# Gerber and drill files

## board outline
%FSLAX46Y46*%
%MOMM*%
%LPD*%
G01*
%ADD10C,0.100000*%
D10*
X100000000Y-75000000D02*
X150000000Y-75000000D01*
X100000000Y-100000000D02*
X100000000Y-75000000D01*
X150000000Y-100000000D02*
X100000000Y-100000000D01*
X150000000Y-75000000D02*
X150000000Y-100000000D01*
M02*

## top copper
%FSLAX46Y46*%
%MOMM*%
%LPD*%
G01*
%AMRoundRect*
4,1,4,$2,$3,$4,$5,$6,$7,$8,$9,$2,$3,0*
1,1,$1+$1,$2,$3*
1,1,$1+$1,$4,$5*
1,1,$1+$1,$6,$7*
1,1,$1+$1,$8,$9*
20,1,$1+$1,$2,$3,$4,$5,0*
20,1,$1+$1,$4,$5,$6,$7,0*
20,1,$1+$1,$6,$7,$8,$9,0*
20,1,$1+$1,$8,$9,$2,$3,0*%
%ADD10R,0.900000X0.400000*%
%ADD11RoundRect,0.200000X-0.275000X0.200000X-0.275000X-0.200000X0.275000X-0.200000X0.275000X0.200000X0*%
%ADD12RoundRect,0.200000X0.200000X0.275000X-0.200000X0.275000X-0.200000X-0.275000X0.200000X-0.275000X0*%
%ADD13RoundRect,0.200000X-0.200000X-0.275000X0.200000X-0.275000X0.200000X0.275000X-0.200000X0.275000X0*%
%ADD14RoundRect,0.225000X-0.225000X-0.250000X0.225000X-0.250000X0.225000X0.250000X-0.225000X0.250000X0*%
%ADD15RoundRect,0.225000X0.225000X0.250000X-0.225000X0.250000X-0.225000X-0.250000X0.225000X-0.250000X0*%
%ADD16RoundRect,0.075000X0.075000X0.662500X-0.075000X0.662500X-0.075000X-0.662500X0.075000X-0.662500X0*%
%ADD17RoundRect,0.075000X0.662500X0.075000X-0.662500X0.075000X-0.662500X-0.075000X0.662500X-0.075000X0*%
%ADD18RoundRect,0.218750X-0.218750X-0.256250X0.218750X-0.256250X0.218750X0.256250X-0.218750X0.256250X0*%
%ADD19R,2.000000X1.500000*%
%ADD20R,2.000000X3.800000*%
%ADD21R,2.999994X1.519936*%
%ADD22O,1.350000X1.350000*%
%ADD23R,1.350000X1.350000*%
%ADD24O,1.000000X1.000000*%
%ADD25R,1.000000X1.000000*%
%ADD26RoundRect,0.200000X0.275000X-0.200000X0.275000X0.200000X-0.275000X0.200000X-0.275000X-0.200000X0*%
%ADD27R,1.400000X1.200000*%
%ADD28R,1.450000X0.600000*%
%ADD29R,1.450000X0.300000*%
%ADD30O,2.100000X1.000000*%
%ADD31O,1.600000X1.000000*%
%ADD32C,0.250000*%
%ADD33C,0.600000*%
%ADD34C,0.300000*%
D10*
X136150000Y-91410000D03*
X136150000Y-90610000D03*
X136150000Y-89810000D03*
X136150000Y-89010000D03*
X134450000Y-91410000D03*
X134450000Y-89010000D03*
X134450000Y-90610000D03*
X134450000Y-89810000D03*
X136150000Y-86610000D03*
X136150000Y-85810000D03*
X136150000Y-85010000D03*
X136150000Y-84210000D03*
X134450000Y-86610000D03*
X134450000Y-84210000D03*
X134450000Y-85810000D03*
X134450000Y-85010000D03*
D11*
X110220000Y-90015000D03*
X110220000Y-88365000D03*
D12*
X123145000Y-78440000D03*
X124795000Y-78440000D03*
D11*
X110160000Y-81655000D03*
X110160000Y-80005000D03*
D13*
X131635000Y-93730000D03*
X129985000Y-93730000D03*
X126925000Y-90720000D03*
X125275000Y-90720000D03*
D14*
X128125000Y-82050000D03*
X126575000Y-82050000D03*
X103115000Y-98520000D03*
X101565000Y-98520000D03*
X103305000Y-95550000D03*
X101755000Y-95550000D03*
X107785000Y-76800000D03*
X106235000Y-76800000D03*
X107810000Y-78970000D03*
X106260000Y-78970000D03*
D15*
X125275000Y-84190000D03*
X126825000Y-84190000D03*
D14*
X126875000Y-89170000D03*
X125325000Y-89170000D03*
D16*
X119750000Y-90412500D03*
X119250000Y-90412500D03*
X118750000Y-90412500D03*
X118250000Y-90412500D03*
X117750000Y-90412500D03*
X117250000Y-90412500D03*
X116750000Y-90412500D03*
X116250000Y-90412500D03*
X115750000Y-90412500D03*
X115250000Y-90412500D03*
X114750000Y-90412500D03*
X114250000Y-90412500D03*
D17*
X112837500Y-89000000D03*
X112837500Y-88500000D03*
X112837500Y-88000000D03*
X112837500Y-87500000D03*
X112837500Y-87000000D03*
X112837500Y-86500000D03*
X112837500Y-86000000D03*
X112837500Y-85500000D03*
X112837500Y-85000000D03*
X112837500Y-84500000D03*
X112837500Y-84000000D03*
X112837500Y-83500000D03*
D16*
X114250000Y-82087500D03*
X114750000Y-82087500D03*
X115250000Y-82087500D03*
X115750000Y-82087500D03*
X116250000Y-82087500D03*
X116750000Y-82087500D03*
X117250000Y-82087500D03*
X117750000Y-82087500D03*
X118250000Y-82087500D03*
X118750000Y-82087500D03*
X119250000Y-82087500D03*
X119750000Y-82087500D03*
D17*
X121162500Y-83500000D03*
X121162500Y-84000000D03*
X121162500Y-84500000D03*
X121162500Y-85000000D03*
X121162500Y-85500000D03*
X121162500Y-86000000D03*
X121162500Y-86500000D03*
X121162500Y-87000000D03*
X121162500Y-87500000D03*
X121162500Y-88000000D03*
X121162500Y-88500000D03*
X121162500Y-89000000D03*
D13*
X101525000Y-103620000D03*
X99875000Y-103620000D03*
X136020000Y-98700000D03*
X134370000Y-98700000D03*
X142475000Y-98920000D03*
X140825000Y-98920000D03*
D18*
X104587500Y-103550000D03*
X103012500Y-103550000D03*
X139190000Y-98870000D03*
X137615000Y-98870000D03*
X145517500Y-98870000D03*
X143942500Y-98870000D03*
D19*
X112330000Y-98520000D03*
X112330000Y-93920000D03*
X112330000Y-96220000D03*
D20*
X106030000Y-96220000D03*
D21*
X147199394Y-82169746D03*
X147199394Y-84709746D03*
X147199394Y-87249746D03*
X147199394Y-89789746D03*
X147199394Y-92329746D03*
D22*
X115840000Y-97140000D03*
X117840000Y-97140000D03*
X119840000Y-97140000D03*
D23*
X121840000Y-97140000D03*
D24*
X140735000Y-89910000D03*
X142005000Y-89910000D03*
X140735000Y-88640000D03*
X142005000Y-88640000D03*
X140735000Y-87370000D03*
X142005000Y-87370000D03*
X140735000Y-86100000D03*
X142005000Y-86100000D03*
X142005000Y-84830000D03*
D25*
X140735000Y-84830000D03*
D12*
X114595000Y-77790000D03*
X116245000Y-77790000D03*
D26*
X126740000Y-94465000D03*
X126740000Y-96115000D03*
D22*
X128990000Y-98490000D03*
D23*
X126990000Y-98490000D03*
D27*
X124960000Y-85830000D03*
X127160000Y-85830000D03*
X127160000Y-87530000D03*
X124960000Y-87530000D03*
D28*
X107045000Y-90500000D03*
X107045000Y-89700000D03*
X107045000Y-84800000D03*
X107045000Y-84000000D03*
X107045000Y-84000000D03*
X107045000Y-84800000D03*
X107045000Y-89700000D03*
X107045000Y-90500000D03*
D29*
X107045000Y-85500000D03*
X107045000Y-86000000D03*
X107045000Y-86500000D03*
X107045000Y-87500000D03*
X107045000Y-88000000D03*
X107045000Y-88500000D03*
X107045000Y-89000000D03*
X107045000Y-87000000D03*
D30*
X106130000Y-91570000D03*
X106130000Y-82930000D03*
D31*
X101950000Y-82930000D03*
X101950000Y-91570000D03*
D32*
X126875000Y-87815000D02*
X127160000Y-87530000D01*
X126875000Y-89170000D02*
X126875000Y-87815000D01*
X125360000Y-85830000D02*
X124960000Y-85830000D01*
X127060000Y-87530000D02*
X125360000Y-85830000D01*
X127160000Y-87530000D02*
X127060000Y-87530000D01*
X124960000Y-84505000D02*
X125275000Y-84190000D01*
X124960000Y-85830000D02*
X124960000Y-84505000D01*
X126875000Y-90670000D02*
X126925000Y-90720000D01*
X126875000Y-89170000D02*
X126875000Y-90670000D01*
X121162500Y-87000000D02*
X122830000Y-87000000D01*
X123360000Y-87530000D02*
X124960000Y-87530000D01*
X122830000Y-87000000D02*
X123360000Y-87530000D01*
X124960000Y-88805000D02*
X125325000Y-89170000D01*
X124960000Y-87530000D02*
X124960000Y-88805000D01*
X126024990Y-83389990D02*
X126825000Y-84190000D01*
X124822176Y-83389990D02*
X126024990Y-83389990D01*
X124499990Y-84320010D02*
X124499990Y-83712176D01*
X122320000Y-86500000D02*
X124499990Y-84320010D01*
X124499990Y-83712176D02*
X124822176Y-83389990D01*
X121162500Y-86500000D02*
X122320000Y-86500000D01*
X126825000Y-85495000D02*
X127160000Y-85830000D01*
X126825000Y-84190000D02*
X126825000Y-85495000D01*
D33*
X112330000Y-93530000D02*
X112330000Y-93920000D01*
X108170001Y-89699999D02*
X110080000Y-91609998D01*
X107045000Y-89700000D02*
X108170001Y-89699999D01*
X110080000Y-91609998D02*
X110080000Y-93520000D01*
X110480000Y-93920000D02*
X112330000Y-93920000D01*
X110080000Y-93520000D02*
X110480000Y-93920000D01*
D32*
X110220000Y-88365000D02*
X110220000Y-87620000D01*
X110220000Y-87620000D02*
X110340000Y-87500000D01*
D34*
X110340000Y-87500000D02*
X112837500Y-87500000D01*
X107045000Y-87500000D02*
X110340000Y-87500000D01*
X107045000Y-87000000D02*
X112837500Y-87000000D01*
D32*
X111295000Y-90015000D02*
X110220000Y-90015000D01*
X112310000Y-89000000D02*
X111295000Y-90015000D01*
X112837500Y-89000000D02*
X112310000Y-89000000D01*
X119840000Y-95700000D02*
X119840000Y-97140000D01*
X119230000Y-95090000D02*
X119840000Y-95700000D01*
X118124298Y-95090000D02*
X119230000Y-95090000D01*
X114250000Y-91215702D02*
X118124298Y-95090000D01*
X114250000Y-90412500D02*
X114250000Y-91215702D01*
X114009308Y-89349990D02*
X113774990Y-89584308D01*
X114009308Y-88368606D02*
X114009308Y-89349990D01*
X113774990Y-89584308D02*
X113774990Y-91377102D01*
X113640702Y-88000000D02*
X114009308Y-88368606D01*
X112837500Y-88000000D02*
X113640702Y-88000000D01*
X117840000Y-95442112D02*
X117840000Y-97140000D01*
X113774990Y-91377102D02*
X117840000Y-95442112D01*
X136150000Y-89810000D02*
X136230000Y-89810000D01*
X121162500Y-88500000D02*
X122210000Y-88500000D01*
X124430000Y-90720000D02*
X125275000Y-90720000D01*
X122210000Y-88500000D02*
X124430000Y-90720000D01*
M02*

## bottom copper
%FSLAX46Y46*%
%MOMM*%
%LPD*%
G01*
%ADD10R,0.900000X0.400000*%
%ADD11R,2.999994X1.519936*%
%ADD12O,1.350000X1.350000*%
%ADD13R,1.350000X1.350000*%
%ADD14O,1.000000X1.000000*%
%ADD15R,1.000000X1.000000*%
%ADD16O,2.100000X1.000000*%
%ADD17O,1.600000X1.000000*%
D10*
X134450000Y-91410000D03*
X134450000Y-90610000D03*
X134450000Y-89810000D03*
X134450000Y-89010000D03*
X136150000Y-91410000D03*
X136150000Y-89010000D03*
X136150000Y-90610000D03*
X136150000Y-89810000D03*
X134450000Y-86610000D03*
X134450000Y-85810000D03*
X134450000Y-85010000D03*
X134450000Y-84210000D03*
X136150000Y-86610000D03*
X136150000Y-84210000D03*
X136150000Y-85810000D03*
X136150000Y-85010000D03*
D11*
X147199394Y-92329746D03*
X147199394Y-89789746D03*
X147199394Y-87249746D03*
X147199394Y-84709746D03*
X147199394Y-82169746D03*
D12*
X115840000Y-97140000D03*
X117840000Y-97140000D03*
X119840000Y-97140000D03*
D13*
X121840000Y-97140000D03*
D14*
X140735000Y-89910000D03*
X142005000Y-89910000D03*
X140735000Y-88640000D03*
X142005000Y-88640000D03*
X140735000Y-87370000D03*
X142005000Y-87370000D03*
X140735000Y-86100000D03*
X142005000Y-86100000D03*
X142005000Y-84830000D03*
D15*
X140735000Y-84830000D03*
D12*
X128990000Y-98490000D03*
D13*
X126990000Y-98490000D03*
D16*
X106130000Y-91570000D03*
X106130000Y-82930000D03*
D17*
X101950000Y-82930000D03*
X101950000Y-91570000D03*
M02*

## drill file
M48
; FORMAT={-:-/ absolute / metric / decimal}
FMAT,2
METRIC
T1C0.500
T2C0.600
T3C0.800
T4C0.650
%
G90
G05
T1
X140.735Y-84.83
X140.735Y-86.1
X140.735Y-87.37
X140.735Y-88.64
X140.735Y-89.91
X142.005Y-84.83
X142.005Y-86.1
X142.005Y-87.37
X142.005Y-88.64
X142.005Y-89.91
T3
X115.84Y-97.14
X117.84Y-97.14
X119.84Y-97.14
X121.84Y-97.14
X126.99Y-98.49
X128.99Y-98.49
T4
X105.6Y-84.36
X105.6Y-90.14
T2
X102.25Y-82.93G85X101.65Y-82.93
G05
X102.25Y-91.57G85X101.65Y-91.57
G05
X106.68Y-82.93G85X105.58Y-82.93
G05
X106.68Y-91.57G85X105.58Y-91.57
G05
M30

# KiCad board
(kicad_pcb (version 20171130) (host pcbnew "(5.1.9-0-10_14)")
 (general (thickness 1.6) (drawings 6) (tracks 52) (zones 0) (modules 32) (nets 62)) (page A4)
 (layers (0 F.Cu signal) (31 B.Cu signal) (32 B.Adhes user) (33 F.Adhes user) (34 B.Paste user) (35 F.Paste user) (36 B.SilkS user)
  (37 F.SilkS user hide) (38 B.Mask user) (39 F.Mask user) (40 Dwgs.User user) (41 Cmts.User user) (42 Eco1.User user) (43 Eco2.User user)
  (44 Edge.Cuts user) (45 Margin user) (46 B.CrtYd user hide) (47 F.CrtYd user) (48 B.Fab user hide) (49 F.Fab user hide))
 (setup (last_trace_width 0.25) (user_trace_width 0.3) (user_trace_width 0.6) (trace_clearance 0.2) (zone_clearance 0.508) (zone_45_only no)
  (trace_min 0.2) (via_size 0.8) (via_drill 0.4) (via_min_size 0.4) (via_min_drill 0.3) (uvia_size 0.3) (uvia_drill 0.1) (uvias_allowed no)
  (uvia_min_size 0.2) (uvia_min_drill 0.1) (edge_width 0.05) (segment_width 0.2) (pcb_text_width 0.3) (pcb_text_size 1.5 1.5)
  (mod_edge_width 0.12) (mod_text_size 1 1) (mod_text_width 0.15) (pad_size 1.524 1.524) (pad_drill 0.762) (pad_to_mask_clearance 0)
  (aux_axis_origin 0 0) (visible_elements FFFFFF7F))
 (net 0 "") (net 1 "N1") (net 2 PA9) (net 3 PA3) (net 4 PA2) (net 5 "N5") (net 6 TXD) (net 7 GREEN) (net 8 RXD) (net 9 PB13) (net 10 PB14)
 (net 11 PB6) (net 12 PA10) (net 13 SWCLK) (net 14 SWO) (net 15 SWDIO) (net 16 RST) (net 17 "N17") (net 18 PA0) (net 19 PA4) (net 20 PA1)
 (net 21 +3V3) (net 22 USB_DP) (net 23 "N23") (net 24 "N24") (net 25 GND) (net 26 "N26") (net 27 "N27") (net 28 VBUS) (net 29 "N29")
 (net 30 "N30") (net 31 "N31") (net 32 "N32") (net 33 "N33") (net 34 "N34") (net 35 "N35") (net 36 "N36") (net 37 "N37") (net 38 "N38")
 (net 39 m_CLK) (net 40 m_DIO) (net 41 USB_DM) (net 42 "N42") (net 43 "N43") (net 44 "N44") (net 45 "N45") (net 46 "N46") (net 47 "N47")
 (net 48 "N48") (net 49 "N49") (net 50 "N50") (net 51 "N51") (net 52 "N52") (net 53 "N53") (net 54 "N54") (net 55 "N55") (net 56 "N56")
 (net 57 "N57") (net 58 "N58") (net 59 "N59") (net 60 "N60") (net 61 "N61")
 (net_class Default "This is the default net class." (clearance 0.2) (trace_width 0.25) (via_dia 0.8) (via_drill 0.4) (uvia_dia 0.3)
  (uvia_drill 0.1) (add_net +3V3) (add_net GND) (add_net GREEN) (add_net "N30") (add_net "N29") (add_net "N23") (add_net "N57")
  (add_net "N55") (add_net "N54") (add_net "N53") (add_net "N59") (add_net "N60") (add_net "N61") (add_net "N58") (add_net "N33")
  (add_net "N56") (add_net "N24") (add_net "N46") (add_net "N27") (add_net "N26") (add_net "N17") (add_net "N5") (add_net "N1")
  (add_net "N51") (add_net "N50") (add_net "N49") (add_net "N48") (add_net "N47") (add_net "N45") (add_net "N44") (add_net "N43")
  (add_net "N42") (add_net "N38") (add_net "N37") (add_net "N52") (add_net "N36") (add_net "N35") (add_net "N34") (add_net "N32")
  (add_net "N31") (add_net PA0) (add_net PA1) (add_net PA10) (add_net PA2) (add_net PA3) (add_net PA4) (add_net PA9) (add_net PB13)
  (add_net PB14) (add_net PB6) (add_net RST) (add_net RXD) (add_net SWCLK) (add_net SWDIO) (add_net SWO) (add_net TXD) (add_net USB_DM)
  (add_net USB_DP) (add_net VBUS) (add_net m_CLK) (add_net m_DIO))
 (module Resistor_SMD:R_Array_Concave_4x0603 (layer B.Cu) (at 135.3 90.21 180)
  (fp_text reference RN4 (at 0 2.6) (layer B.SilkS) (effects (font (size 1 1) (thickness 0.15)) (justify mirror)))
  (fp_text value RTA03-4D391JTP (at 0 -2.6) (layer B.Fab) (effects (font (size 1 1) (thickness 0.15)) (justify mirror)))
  (pad 5 smd rect (at 0.85 -1.2 180) (size 0.9 0.4) (layers B.Cu B.Paste B.Mask) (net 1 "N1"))
  (pad 6 smd rect (at 0.85 -0.4 180) (size 0.9 0.4) (layers B.Cu B.Paste B.Mask) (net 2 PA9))
  (pad 7 smd rect (at 0.85 0.4 180) (size 0.9 0.4) (layers B.Cu B.Paste B.Mask) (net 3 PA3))
  (pad 8 smd rect (at 0.85 1.2 180) (size 0.9 0.4) (layers B.Cu B.Paste B.Mask) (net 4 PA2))
  (pad 4 smd rect (at -0.85 -1.2 180) (size 0.9 0.4) (layers B.Cu B.Paste B.Mask) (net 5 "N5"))
  (pad 1 smd rect (at -0.85 1.2 180) (size 0.9 0.4) (layers B.Cu B.Paste B.Mask) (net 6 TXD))
  (pad 3 smd rect (at -0.85 -0.4 180) (size 0.9 0.4) (layers B.Cu B.Paste B.Mask) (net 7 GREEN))
  (pad 2 smd rect (at -0.85 0.4 180) (size 0.9 0.4) (layers B.Cu B.Paste B.Mask) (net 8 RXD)))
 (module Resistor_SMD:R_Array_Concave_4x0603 (layer B.Cu) (at 135.3 85.41 180)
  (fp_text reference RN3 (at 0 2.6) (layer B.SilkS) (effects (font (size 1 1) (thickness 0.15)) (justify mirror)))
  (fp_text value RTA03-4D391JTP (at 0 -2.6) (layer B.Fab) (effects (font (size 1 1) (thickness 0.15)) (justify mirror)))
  (pad 5 smd rect (at 0.85 -1.2 180) (size 0.9 0.4) (layers B.Cu B.Paste B.Mask) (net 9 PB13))
  (pad 6 smd rect (at 0.85 -0.4 180) (size 0.9 0.4) (layers B.Cu B.Paste B.Mask) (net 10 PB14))
  (pad 7 smd rect (at 0.85 0.4 180) (size 0.9 0.4) (layers B.Cu B.Paste B.Mask) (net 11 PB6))
  (pad 8 smd rect (at 0.85 1.2 180) (size 0.9 0.4) (layers B.Cu B.Paste B.Mask) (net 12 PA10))
  (pad 4 smd rect (at -0.85 -1.2 180) (size 0.9 0.4) (layers B.Cu B.Paste B.Mask) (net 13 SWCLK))
  (pad 1 smd rect (at -0.85 1.2 180) (size 0.9 0.4) (layers B.Cu B.Paste B.Mask) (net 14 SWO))
  (pad 3 smd rect (at -0.85 -0.4 180) (size 0.9 0.4) (layers B.Cu B.Paste B.Mask) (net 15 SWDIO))
  (pad 2 smd rect (at -0.85 0.4 180) (size 0.9 0.4) (layers B.Cu B.Paste B.Mask) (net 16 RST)))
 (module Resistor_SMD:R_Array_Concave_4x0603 (layer F.Cu) (at 135.3 90.21)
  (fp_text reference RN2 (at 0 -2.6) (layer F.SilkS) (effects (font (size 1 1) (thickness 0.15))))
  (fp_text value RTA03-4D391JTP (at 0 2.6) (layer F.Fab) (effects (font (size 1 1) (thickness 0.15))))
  (pad 5 smd rect (at 0.85 1.2) (size 0.9 0.4) (layers F.Cu F.Paste F.Mask) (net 5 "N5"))
  (pad 6 smd rect (at 0.85 0.4) (size 0.9 0.4) (layers F.Cu F.Paste F.Mask) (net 7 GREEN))
  (pad 7 smd rect (at 0.85 -0.4) (size 0.9 0.4) (layers F.Cu F.Paste F.Mask) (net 8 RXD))
  (pad 8 smd rect (at 0.85 -1.2) (size 0.9 0.4) (layers F.Cu F.Paste F.Mask) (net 6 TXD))
  (pad 4 smd rect (at -0.85 1.2) (size 0.9 0.4) (layers F.Cu F.Paste F.Mask) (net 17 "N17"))
  (pad 1 smd rect (at -0.85 -1.2) (size 0.9 0.4) (layers F.Cu F.Paste F.Mask) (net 2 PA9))
  (pad 3 smd rect (at -0.85 0.4) (size 0.9 0.4) (layers F.Cu F.Paste F.Mask) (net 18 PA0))
  (pad 2 smd rect (at -0.85 -0.4) (size 0.9 0.4) (layers F.Cu F.Paste F.Mask) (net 12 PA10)))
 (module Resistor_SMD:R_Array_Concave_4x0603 (layer F.Cu) (at 135.3 85.41)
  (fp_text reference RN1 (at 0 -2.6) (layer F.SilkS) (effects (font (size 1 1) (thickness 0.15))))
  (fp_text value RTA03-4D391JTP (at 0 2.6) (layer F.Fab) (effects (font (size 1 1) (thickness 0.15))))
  (pad 5 smd rect (at 0.85 1.2) (size 0.9 0.4) (layers F.Cu F.Paste F.Mask) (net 13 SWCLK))
  (pad 6 smd rect (at 0.85 0.4) (size 0.9 0.4) (layers F.Cu F.Paste F.Mask) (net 15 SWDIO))
  (pad 7 smd rect (at 0.85 -0.4) (size 0.9 0.4) (layers F.Cu F.Paste F.Mask) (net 16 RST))
  (pad 8 smd rect (at 0.85 -1.2) (size 0.9 0.4) (layers F.Cu F.Paste F.Mask) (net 14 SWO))
  (pad 4 smd rect (at -0.85 1.2) (size 0.9 0.4) (layers F.Cu F.Paste F.Mask) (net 4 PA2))
  (pad 1 smd rect (at -0.85 -1.2) (size 0.9 0.4) (layers F.Cu F.Paste F.Mask) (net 3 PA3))
  (pad 3 smd rect (at -0.85 0.4) (size 0.9 0.4) (layers F.Cu F.Paste F.Mask) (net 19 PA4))
  (pad 2 smd rect (at -0.85 -0.4) (size 0.9 0.4) (layers F.Cu F.Paste F.Mask) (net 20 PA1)))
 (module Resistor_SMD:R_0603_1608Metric (layer F.Cu) (at 110.22 89.19 270)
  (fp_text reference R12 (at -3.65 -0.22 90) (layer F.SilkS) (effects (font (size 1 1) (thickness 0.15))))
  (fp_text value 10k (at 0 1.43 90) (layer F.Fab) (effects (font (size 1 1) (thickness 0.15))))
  (pad 2 smd roundrect (at 0.825 0 270) (size 0.8 0.95) (layers F.Cu F.Paste F.Mask) (roundrect_rratio 0.25) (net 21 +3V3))
  (pad 1 smd roundrect (at -0.825 0 270) (size 0.8 0.95) (layers F.Cu F.Paste F.Mask) (roundrect_rratio 0.25) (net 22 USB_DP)))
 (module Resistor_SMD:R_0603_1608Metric (layer F.Cu) (at 123.97 78.44 180)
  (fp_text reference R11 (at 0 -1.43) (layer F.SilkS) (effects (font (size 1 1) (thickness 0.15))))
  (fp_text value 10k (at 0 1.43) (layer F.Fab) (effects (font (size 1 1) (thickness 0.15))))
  (pad 2 smd roundrect (at 0.825 0 180) (size 0.8 0.95) (layers F.Cu F.Paste F.Mask) (roundrect_rratio 0.25) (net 21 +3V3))
  (pad 1 smd roundrect (at -0.825 0 180) (size 0.8 0.95) (layers F.Cu F.Paste F.Mask) (roundrect_rratio 0.25) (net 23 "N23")))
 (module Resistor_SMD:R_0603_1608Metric (layer F.Cu) (at 110.16 80.83 270)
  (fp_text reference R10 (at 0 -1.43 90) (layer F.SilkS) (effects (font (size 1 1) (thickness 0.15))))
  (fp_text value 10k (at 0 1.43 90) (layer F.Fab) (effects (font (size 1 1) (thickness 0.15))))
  (pad 2 smd roundrect (at 0.825 0 270) (size 0.8 0.95) (layers F.Cu F.Paste F.Mask) (roundrect_rratio 0.25) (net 10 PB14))
  (pad 1 smd roundrect (at -0.825 0 270) (size 0.8 0.95) (layers F.Cu F.Paste F.Mask) (roundrect_rratio 0.25) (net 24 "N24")))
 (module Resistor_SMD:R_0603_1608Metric (layer F.Cu) (at 130.81 93.73)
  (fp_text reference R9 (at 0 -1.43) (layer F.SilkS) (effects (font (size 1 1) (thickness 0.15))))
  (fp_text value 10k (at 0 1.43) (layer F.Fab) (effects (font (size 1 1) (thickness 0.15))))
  (pad 2 smd roundrect (at 0.825 0) (size 0.8 0.95) (layers F.Cu F.Paste F.Mask) (roundrect_rratio 0.25) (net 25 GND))
  (pad 1 smd roundrect (at -0.825 0) (size 0.8 0.95) (layers F.Cu F.Paste F.Mask) (roundrect_rratio 0.25) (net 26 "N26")))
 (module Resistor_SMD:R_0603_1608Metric (layer F.Cu) (at 126.1 90.72)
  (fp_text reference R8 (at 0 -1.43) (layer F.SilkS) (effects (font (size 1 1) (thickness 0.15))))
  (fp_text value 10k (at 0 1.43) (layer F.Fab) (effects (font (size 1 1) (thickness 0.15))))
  (pad 2 smd roundrect (at 0.825 0) (size 0.8 0.95) (layers F.Cu F.Paste F.Mask) (roundrect_rratio 0.25) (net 25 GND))
  (pad 1 smd roundrect (at -0.825 0) (size 0.8 0.95) (layers F.Cu F.Paste F.Mask) (roundrect_rratio 0.25) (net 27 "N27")))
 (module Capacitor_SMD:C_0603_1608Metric (layer F.Cu) (at 127.35 82.05)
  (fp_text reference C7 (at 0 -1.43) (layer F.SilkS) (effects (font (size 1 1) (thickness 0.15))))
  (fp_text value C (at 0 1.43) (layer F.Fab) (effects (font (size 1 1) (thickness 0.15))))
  (pad 2 smd roundrect (at 0.775 0) (size 0.9 0.95) (layers F.Cu F.Paste F.Mask) (roundrect_rratio 0.25) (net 25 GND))
  (pad 1 smd roundrect (at -0.775 0) (size 0.9 0.95) (layers F.Cu F.Paste F.Mask) (roundrect_rratio 0.25) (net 23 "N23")))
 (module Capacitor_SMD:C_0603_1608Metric (layer F.Cu) (at 102.34 98.52)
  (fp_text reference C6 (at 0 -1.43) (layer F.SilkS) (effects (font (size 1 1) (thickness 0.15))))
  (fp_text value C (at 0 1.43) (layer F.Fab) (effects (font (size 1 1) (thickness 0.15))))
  (pad 2 smd roundrect (at 0.775 0) (size 0.9 0.95) (layers F.Cu F.Paste F.Mask) (roundrect_rratio 0.25) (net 21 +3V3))
  (pad 1 smd roundrect (at -0.775 0) (size 0.9 0.95) (layers F.Cu F.Paste F.Mask) (roundrect_rratio 0.25) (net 25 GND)))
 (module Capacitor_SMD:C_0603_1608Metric (layer F.Cu) (at 102.53 95.55)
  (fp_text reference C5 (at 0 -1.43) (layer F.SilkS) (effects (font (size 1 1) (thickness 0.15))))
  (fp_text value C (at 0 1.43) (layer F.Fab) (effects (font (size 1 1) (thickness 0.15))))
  (pad 2 smd roundrect (at 0.775 0) (size 0.9 0.95) (layers F.Cu F.Paste F.Mask) (roundrect_rratio 0.25) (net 21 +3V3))
  (pad 1 smd roundrect (at -0.775 0) (size 0.9 0.95) (layers F.Cu F.Paste F.Mask) (roundrect_rratio 0.25) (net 25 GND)))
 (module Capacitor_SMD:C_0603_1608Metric (layer F.Cu) (at 107.01 76.8)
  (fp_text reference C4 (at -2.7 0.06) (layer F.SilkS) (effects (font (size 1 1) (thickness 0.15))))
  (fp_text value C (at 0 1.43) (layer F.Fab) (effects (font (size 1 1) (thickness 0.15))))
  (pad 2 smd roundrect (at 0.775 0) (size 0.9 0.95) (layers F.Cu F.Paste F.Mask) (roundrect_rratio 0.25) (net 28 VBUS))
  (pad 1 smd roundrect (at -0.775 0) (size 0.9 0.95) (layers F.Cu F.Paste F.Mask) (roundrect_rratio 0.25) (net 25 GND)))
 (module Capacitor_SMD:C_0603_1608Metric (layer F.Cu) (at 107.035 78.97)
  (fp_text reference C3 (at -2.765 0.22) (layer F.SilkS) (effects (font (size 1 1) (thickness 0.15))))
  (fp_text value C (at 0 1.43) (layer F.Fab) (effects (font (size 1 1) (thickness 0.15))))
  (pad 2 smd roundrect (at 0.775 0) (size 0.9 0.95) (layers F.Cu F.Paste F.Mask) (roundrect_rratio 0.25) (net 28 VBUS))
  (pad 1 smd roundrect (at -0.775 0) (size 0.9 0.95) (layers F.Cu F.Paste F.Mask) (roundrect_rratio 0.25) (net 25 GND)))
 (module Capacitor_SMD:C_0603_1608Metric (layer F.Cu) (at 126.05 84.19 180)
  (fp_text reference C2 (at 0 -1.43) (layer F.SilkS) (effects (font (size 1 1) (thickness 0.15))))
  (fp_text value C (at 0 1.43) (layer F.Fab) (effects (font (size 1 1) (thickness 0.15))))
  (pad 2 smd roundrect (at 0.775 0 180) (size 0.9 0.95) (layers F.Cu F.Paste F.Mask) (roundrect_rratio 0.25) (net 25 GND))
  (pad 1 smd roundrect (at -0.775 0 180) (size 0.9 0.95) (layers F.Cu F.Paste F.Mask) (roundrect_rratio 0.25) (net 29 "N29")))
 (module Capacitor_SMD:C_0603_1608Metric (layer F.Cu) (at 126.1 89.17)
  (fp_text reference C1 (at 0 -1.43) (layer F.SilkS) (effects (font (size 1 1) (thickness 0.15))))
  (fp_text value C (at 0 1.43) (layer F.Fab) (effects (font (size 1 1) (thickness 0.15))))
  (pad 2 smd roundrect (at 0.775 0) (size 0.9 0.95) (layers F.Cu F.Paste F.Mask) (roundrect_rratio 0.25) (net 25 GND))
  (pad 1 smd roundrect (at -0.775 0) (size 0.9 0.95) (layers F.Cu F.Paste F.Mask) (roundrect_rratio 0.25) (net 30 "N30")))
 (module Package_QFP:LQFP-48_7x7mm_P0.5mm (layer F.Cu) (at 117 86.25 180)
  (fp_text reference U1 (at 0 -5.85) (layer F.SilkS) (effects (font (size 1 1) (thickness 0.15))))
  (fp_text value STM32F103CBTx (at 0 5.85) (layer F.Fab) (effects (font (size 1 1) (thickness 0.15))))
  (pad 48 smd roundrect (at -2.75 -4.1625 180) (size 0.3 1.475) (layers F.Cu F.Paste F.Mask) (roundrect_rratio 0.25) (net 21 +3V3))
  (pad 47 smd roundrect (at -2.25 -4.1625 180) (size 0.3 1.475) (layers F.Cu F.Paste F.Mask) (roundrect_rratio 0.25) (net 25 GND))
  (pad 46 smd roundrect (at -1.75 -4.1625 180) (size 0.3 1.475) (layers F.Cu F.Paste F.Mask) (roundrect_rratio 0.25) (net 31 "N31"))
  (pad 45 smd roundrect (at -1.25 -4.1625 180) (size 0.3 1.475) (layers F.Cu F.Paste F.Mask) (roundrect_rratio 0.25) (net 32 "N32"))
  (pad 44 smd roundrect (at -0.75 -4.1625 180) (size 0.3 1.475) (layers F.Cu F.Paste F.Mask) (roundrect_rratio 0.25) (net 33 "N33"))
  (pad 43 smd roundrect (at -0.25 -4.1625 180) (size 0.3 1.475) (layers F.Cu F.Paste F.Mask) (roundrect_rratio 0.25) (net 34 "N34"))
  (pad 42 smd roundrect (at 0.25 -4.1625 180) (size 0.3 1.475) (layers F.Cu F.Paste F.Mask) (roundrect_rratio 0.25) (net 11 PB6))
  (pad 41 smd roundrect (at 0.75 -4.1625 180) (size 0.3 1.475) (layers F.Cu F.Paste F.Mask) (roundrect_rratio 0.25) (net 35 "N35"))
  (pad 40 smd roundrect (at 1.25 -4.1625 180) (size 0.3 1.475) (layers F.Cu F.Paste F.Mask) (roundrect_rratio 0.25) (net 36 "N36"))
  (pad 39 smd roundrect (at 1.75 -4.1625 180) (size 0.3 1.475) (layers F.Cu F.Paste F.Mask) (roundrect_rratio 0.25) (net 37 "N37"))
  (pad 38 smd roundrect (at 2.25 -4.1625 180) (size 0.3 1.475) (layers F.Cu F.Paste F.Mask) (roundrect_rratio 0.25) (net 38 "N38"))
  (pad 37 smd roundrect (at 2.75 -4.1625 180) (size 0.3 1.475) (layers F.Cu F.Paste F.Mask) (roundrect_rratio 0.25) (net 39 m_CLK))
  (pad 36 smd roundrect (at 4.1625 -2.75 180) (size 1.475 0.3) (layers F.Cu F.Paste F.Mask) (roundrect_rratio 0.25) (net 21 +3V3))
  (pad 35 smd roundrect (at 4.1625 -2.25 180) (size 1.475 0.3) (layers F.Cu F.Paste F.Mask) (roundrect_rratio 0.25) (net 25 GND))
  (pad 34 smd roundrect (at 4.1625 -1.75 180) (size 1.475 0.3) (layers F.Cu F.Paste F.Mask) (roundrect_rratio 0.25) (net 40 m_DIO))
  (pad 33 smd roundrect (at 4.1625 -1.25 180) (size 1.475 0.3) (layers F.Cu F.Paste F.Mask) (roundrect_rratio 0.25) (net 22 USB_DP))
  (pad 32 smd roundrect (at 4.1625 -0.75 180) (size 1.475 0.3) (layers F.Cu F.Paste F.Mask) (roundrect_rratio 0.25) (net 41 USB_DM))
  (pad 31 smd roundrect (at 4.1625 -0.25 180) (size 1.475 0.3) (layers F.Cu F.Paste F.Mask) (roundrect_rratio 0.25) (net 12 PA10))
  (pad 30 smd roundrect (at 4.1625 0.25 180) (size 1.475 0.3) (layers F.Cu F.Paste F.Mask) (roundrect_rratio 0.25) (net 2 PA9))
  (pad 29 smd roundrect (at 4.1625 0.75 180) (size 1.475 0.3) (layers F.Cu F.Paste F.Mask) (roundrect_rratio 0.25) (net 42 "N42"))
  (pad 28 smd roundrect (at 4.1625 1.25 180) (size 1.475 0.3) (layers F.Cu F.Paste F.Mask) (roundrect_rratio 0.25) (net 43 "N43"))
  (pad 27 smd roundrect (at 4.1625 1.75 180) (size 1.475 0.3) (layers F.Cu F.Paste F.Mask) (roundrect_rratio 0.25) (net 10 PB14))
  (pad 26 smd roundrect (at 4.1625 2.25 180) (size 1.475 0.3) (layers F.Cu F.Paste F.Mask) (roundrect_rratio 0.25) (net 9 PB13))
  (pad 25 smd roundrect (at 4.1625 2.75 180) (size 1.475 0.3) (layers F.Cu F.Paste F.Mask) (roundrect_rratio 0.25) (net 24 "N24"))
  (pad 24 smd roundrect (at 2.75 4.1625 180) (size 0.3 1.475) (layers F.Cu F.Paste F.Mask) (roundrect_rratio 0.25) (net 21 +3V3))
  (pad 23 smd roundrect (at 2.25 4.1625 180) (size 0.3 1.475) (layers F.Cu F.Paste F.Mask) (roundrect_rratio 0.25) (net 25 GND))
  (pad 22 smd roundrect (at 1.75 4.1625 180) (size 0.3 1.475) (layers F.Cu F.Paste F.Mask) (roundrect_rratio 0.25) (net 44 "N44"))
  (pad 21 smd roundrect (at 1.25 4.1625 180) (size 0.3 1.475) (layers F.Cu F.Paste F.Mask) (roundrect_rratio 0.25) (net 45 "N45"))
  (pad 20 smd roundrect (at 0.75 4.1625 180) (size 0.3 1.475) (layers F.Cu F.Paste F.Mask) (roundrect_rratio 0.25) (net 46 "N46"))
  (pad 19 smd roundrect (at 0.25 4.1625 180) (size 0.3 1.475) (layers F.Cu F.Paste F.Mask) (roundrect_rratio 0.25) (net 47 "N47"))
  (pad 18 smd roundrect (at -0.25 4.1625 180) (size 0.3 1.475) (layers F.Cu F.Paste F.Mask) (roundrect_rratio 0.25) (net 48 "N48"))
  (pad 17 smd roundrect (at -0.75 4.1625 180) (size 0.3 1.475) (layers F.Cu F.Paste F.Mask) (roundrect_rratio 0.25) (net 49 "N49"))
  (pad 16 smd roundrect (at -1.25 4.1625 180) (size 0.3 1.475) (layers F.Cu F.Paste F.Mask) (roundrect_rratio 0.25) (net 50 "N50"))
  (pad 15 smd roundrect (at -1.75 4.1625 180) (size 0.3 1.475) (layers F.Cu F.Paste F.Mask) (roundrect_rratio 0.25) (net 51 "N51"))
  (pad 14 smd roundrect (at -2.25 4.1625 180) (size 0.3 1.475) (layers F.Cu F.Paste F.Mask) (roundrect_rratio 0.25) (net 19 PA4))
  (pad 13 smd roundrect (at -2.75 4.1625 180) (size 0.3 1.475) (layers F.Cu F.Paste F.Mask) (roundrect_rratio 0.25) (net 3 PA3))
  (pad 12 smd roundrect (at -4.1625 2.75 180) (size 1.475 0.3) (layers F.Cu F.Paste F.Mask) (roundrect_rratio 0.25) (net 4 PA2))
  (pad 11 smd roundrect (at -4.1625 2.25 180) (size 1.475 0.3) (layers F.Cu F.Paste F.Mask) (roundrect_rratio 0.25) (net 20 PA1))
  (pad 10 smd roundrect (at -4.1625 1.75 180) (size 1.475 0.3) (layers F.Cu F.Paste F.Mask) (roundrect_rratio 0.25) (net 18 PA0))
  (pad 9 smd roundrect (at -4.1625 1.25 180) (size 1.475 0.3) (layers F.Cu F.Paste F.Mask) (roundrect_rratio 0.25) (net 21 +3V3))
  (pad 8 smd roundrect (at -4.1625 0.75 180) (size 1.475 0.3) (layers F.Cu F.Paste F.Mask) (roundrect_rratio 0.25) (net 25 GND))
  (pad 7 smd roundrect (at -4.1625 0.25 180) (size 1.475 0.3) (layers F.Cu F.Paste F.Mask) (roundrect_rratio 0.25) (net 23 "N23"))
  (pad 6 smd roundrect (at -4.1625 -0.25 180) (size 1.475 0.3) (layers F.Cu F.Paste F.Mask) (roundrect_rratio 0.25) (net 29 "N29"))
  (pad 5 smd roundrect (at -4.1625 -0.75 180) (size 1.475 0.3) (layers F.Cu F.Paste F.Mask) (roundrect_rratio 0.25) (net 30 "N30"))
  (pad 4 smd roundrect (at -4.1625 -1.25 180) (size 1.475 0.3) (layers F.Cu F.Paste F.Mask) (roundrect_rratio 0.25) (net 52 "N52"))
  (pad 3 smd roundrect (at -4.1625 -1.75 180) (size 1.475 0.3) (layers F.Cu F.Paste F.Mask) (roundrect_rratio 0.25) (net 26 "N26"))
  (pad 2 smd roundrect (at -4.1625 -2.25 180) (size 1.475 0.3) (layers F.Cu F.Paste F.Mask) (roundrect_rratio 0.25) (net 27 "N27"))
  (pad 1 smd roundrect (at -4.1625 -2.75 180) (size 1.475 0.3) (layers F.Cu F.Paste F.Mask) (roundrect_rratio 0.25) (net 21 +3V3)))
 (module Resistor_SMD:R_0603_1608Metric (layer F.Cu) (at 100.7 103.62)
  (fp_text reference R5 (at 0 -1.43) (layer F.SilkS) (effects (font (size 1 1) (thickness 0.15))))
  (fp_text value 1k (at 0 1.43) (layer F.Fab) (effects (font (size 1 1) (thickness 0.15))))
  (pad 2 smd roundrect (at 0.825 0) (size 0.8 0.95) (layers F.Cu F.Paste F.Mask) (roundrect_rratio 0.25) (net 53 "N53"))
  (pad 1 smd roundrect (at -0.825 0) (size 0.8 0.95) (layers F.Cu F.Paste F.Mask) (roundrect_rratio 0.25) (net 25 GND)))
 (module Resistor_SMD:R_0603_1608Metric (layer F.Cu) (at 135.195 98.7)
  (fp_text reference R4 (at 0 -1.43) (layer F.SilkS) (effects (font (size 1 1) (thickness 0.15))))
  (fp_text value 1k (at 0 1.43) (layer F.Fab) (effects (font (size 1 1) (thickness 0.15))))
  (pad 2 smd roundrect (at 0.825 0) (size 0.8 0.95) (layers F.Cu F.Paste F.Mask) (roundrect_rratio 0.25) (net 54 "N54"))
  (pad 1 smd roundrect (at -0.825 0) (size 0.8 0.95) (layers F.Cu F.Paste F.Mask) (roundrect_rratio 0.25) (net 7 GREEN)))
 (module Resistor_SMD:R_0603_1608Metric (layer F.Cu) (at 141.65 98.92)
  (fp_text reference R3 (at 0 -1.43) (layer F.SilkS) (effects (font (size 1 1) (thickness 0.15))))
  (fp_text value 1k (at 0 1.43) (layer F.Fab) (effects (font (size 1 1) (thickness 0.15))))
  (pad 2 smd roundrect (at 0.825 0) (size 0.8 0.95) (layers F.Cu F.Paste F.Mask) (roundrect_rratio 0.25) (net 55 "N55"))
  (pad 1 smd roundrect (at -0.825 0) (size 0.8 0.95) (layers F.Cu F.Paste F.Mask) (roundrect_rratio 0.25) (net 6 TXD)))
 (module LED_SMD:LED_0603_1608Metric (layer F.Cu) (at 103.8 103.55)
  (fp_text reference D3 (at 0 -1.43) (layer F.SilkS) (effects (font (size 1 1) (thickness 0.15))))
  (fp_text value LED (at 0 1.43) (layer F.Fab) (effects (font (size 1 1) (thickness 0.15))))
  (pad 2 smd roundrect (at 0.7875 0) (size 0.875 0.95) (layers F.Cu F.Paste F.Mask) (roundrect_rratio 0.25) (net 21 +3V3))
  (pad 1 smd roundrect (at -0.7875 0) (size 0.875 0.95) (layers F.Cu F.Paste F.Mask) (roundrect_rratio 0.25) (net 53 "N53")))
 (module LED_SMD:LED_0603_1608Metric (layer F.Cu) (at 138.4025 98.87)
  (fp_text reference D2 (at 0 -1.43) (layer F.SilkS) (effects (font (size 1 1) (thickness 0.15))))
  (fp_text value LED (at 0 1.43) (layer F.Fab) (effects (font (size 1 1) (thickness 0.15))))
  (pad 2 smd roundrect (at 0.7875 0) (size 0.875 0.95) (layers F.Cu F.Paste F.Mask) (roundrect_rratio 0.25) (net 21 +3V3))
  (pad 1 smd roundrect (at -0.7875 0) (size 0.875 0.95) (layers F.Cu F.Paste F.Mask) (roundrect_rratio 0.25) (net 54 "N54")))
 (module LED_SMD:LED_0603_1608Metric (layer F.Cu) (at 144.73 98.87)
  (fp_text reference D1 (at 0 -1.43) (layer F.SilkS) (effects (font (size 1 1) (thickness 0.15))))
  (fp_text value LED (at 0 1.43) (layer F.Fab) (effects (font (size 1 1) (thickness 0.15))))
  (pad 2 smd roundrect (at 0.7875 0) (size 0.875 0.95) (layers F.Cu F.Paste F.Mask) (roundrect_rratio 0.25) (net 21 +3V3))
  (pad 1 smd roundrect (at -0.7875 0) (size 0.875 0.95) (layers F.Cu F.Paste F.Mask) (roundrect_rratio 0.25) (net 55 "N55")))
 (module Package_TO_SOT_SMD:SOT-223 (layer F.Cu) (at 109.18 96.22 180)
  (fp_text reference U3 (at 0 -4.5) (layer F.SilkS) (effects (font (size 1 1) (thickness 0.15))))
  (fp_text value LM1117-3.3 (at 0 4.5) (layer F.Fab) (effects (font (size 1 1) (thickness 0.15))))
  (pad 1 smd rect (at -3.15 -2.3 180) (size 2 1.5) (layers F.Cu F.Paste F.Mask) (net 25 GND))
  (pad 3 smd rect (at -3.15 2.3 180) (size 2 1.5) (layers F.Cu F.Paste F.Mask) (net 28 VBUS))
  (pad 2 smd rect (at -3.15 0 180) (size 2 1.5) (layers F.Cu F.Paste F.Mask) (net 21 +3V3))
  (pad 4 smd rect (at 3.15 0 180) (size 2 3.8) (layers F.Cu F.Paste F.Mask)))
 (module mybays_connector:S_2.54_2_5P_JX (layer F.Cu) (at 146.46 87.25 270)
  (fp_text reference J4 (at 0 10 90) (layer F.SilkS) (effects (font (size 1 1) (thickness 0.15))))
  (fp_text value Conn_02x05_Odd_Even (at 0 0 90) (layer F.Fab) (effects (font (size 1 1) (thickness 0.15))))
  (pad 10 smd rect (at 5.079746 -0.739394) (size 2.999994 1.519936) (layers B.Cu B.Paste B.Mask) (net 8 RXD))
  (pad 8 smd rect (at 2.539746 -0.739394) (size 2.999994 1.519936) (layers B.Cu B.Paste B.Mask) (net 6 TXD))
  (pad 6 smd rect (at -0.000254 -0.739394) (size 2.999994 1.519936) (layers B.Cu B.Paste B.Mask) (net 25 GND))
  (pad 4 smd rect (at -2.540254 -0.739394) (size 2.999994 1.519936) (layers B.Cu B.Paste B.Mask) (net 14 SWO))
  (pad 2 smd rect (at -5.080254 -0.739394) (size 2.999994 1.519936) (layers B.Cu B.Paste B.Mask) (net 16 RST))
  (pad 1 smd rect (at -5.080254 -0.739394) (size 2.999994 1.519936) (layers F.Cu F.Paste F.Mask) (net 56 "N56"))
  (pad 3 smd rect (at -2.540254 -0.739394) (size 2.999994 1.519936) (layers F.Cu F.Paste F.Mask) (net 21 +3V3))
  (pad 5 smd rect (at -0.000254 -0.739394) (size 2.999994 1.519936) (layers F.Cu F.Paste F.Mask) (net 15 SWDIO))
  (pad 7 smd rect (at 2.539746 -0.739394) (size 2.999994 1.519936) (layers F.Cu F.Paste F.Mask) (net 13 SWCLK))
  (pad 9 smd rect (at 5.079746 -0.739394) (size 2.999994 1.519936) (layers F.Cu F.Paste F.Mask) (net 25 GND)))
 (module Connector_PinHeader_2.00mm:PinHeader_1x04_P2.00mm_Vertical (layer F.Cu) (at 121.84 97.14 270)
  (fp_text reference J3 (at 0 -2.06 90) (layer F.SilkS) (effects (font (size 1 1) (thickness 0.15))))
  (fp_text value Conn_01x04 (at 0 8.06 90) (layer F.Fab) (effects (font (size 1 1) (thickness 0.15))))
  (pad 4 thru_hole oval (at 0 6 270) (size 1.35 1.35) (drill 0.8) (layers *.Cu *.Mask) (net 21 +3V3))
  (pad 3 thru_hole oval (at 0 4 270) (size 1.35 1.35) (drill 0.8) (layers *.Cu *.Mask) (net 40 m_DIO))
  (pad 2 thru_hole oval (at 0 2 270) (size 1.35 1.35) (drill 0.8) (layers *.Cu *.Mask) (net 39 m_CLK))
  (pad 1 thru_hole rect (at 0 0 270) (size 1.35 1.35) (drill 0.8) (layers *.Cu *.Mask) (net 25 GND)))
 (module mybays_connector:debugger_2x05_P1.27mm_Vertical (layer F.Cu) (at 141.37 87.37)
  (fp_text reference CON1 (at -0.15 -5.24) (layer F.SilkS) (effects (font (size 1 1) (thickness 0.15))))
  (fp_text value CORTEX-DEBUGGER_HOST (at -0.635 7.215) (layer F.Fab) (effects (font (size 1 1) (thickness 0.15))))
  (pad 9 thru_hole oval (at -0.635 2.54) (size 1 1) (drill 0.5) (layers *.Cu *.Mask) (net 25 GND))
  (pad 10 thru_hole oval (at 0.635 2.54) (size 1 1) (drill 0.5) (layers *.Cu *.Mask) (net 8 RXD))
  (pad 7 thru_hole oval (at -0.635 1.27) (size 1 1) (drill 0.5) (layers *.Cu *.Mask) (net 13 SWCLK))
  (pad 8 thru_hole oval (at 0.635 1.27) (size 1 1) (drill 0.5) (layers *.Cu *.Mask) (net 6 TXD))
  (pad 5 thru_hole oval (at -0.635 0) (size 1 1) (drill 0.5) (layers *.Cu *.Mask) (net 15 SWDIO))
  (pad 6 thru_hole oval (at 0.635 0) (size 1 1) (drill 0.5) (layers *.Cu *.Mask) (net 25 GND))
  (pad 3 thru_hole oval (at -0.635 -1.27) (size 1 1) (drill 0.5) (layers *.Cu *.Mask) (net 21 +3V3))
  (pad 4 thru_hole oval (at 0.635 -1.27) (size 1 1) (drill 0.5) (layers *.Cu *.Mask) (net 14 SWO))
  (pad 2 thru_hole oval (at 0.635 -2.54) (size 1 1) (drill 0.5) (layers *.Cu *.Mask) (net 16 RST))
  (pad 1 thru_hole rect (at -0.635 -2.54) (size 1 1) (drill 0.5) (layers *.Cu *.Mask) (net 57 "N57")))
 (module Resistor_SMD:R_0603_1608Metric (layer F.Cu) (at 115.42 77.79 180)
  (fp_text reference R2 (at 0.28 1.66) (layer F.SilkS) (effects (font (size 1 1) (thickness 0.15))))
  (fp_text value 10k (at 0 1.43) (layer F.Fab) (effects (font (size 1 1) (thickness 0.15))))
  (pad 2 smd roundrect (at 0.825 0 180) (size 0.8 0.95) (layers F.Cu F.Paste F.Mask) (roundrect_rratio 0.25) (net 25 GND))
  (pad 1 smd roundrect (at -0.825 0 180) (size 0.8 0.95) (layers F.Cu F.Paste F.Mask) (roundrect_rratio 0.25) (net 46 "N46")))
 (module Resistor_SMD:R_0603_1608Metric (layer F.Cu) (at 126.74 95.29 90)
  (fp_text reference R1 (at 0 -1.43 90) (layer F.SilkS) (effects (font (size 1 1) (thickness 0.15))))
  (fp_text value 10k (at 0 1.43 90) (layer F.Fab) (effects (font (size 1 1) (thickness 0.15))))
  (pad 2 smd roundrect (at 0.825 0 90) (size 0.8 0.95) (layers F.Cu F.Paste F.Mask) (roundrect_rratio 0.25) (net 25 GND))
  (pad 1 smd roundrect (at -0.825 0 90) (size 0.8 0.95) (layers F.Cu F.Paste F.Mask) (roundrect_rratio 0.25) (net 33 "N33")))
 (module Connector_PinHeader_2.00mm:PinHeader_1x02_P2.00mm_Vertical (layer F.Cu) (at 126.99 98.49 90)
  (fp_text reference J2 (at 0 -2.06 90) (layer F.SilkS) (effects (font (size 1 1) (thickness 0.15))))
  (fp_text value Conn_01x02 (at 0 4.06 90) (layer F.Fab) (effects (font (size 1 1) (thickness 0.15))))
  (pad 2 thru_hole oval (at 0 2 90) (size 1.35 1.35) (drill 0.8) (layers *.Cu *.Mask) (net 21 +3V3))
  (pad 1 thru_hole rect (at 0 0 90) (size 1.35 1.35) (drill 0.8) (layers *.Cu *.Mask) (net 33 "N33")))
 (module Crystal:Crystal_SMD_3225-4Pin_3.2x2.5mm (layer F.Cu) (at 126.06 86.68)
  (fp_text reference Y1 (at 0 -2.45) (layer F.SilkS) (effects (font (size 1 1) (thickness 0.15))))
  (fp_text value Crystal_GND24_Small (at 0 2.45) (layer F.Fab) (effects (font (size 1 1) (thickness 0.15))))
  (pad 4 smd rect (at -1.1 -0.85) (size 1.4 1.2) (layers F.Cu F.Paste F.Mask) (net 25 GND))
  (pad 3 smd rect (at 1.1 -0.85) (size 1.4 1.2) (layers F.Cu F.Paste F.Mask) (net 29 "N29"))
  (pad 2 smd rect (at 1.1 0.85) (size 1.4 1.2) (layers F.Cu F.Paste F.Mask) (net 25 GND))
  (pad 1 smd rect (at -1.1 0.85) (size 1.4 1.2) (layers F.Cu F.Paste F.Mask) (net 30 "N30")))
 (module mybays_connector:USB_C (layer F.Cu) (at 103 87.25 270)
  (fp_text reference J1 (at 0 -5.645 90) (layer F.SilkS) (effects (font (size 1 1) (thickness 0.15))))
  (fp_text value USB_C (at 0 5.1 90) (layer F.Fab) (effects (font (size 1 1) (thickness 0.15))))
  (pad B1 smd rect (at 3.25 -4.045 270) (size 0.6 1.45) (layers F.Cu F.Paste F.Mask) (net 25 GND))
  (pad A9 smd rect (at 2.45 -4.045 270) (size 0.6 1.45) (layers F.Cu F.Paste F.Mask) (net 28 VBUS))
  (pad B9 smd rect (at -2.45 -4.045 270) (size 0.6 1.45) (layers F.Cu F.Paste F.Mask) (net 28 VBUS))
  (pad B12 smd rect (at -3.25 -4.045 270) (size 0.6 1.45) (layers F.Cu F.Paste F.Mask) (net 25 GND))
  (pad A1 smd rect (at -3.25 -4.045 270) (size 0.6 1.45) (layers F.Cu F.Paste F.Mask) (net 25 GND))
  (pad A4 smd rect (at -2.45 -4.045 270) (size 0.6 1.45) (layers F.Cu F.Paste F.Mask) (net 28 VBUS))
  (pad B4 smd rect (at 2.45 -4.045 270) (size 0.6 1.45) (layers F.Cu F.Paste F.Mask) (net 28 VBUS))
  (pad A12 smd rect (at 3.25 -4.045 270) (size 0.6 1.45) (layers F.Cu F.Paste F.Mask) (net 25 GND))
  (pad B8 smd rect (at -1.75 -4.045 270) (size 0.3 1.45) (layers F.Cu F.Paste F.Mask) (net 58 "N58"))
  (pad A5 smd rect (at -1.25 -4.045 270) (size 0.3 1.45) (layers F.Cu F.Paste F.Mask) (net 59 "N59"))
  (pad B7 smd rect (at -0.75 -4.045 270) (size 0.3 1.45) (layers F.Cu F.Paste F.Mask) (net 22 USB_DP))
  (pad A7 smd rect (at 0.25 -4.045 270) (size 0.3 1.45) (layers F.Cu F.Paste F.Mask) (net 22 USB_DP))
  (pad B6 smd rect (at 0.75 -4.045 270) (size 0.3 1.45) (layers F.Cu F.Paste F.Mask) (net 41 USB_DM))
  (pad A8 smd rect (at 1.25 -4.045 270) (size 0.3 1.45) (layers F.Cu F.Paste F.Mask) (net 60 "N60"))
  (pad B5 smd rect (at 1.75 -4.045 270) (size 0.3 1.45) (layers F.Cu F.Paste F.Mask) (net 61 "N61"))
  (pad A6 smd rect (at -0.25 -4.045 270) (size 0.3 1.45) (layers F.Cu F.Paste F.Mask) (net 41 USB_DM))
  (pad S1 thru_hole oval (at 4.32 -3.13 270) (size 1 2.1) (drill oval 0.6 1.7) (layers *.Cu *.Mask) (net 25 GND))
  (pad S1 thru_hole oval (at -4.32 -3.13 270) (size 1 2.1) (drill oval 0.6 1.7) (layers *.Cu *.Mask) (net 25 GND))
  (pad "" np_thru_hole circle (at -2.89 -2.6 270) (size 0.65 0.65) (drill 0.65) (layers *.Cu *.Mask))
  (pad S1 thru_hole oval (at -4.32 1.05 270) (size 1 1.6) (drill oval 0.6 1.2) (layers *.Cu *.Mask) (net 25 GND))
  (pad "" np_thru_hole circle (at 2.89 -2.6 270) (size 0.65 0.65) (drill 0.65) (layers *.Cu *.Mask))
  (pad S1 thru_hole oval (at 4.32 1.05 270) (size 1 1.6) (drill oval 0.6 1.2) (layers *.Cu *.Mask) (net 25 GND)))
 (gr_line (start 100 75) (end 150 75) (layer Edge.Cuts) (width 0.1))
 (gr_line (start 100 100) (end 100 75) (layer Edge.Cuts) (width 0.1))
 (gr_line (start 150 100) (end 100 100) (layer Edge.Cuts) (width 0.1))
 (gr_line (start 150 75) (end 150 100) (layer Edge.Cuts) (width 0.1))
 (segment (start 126.875 87.815) (end 127.16 87.53) (width 0.25) (layer F.Cu) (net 25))
 (segment (start 126.875 89.17) (end 126.875 87.815) (width 0.25) (layer F.Cu) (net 25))
 (segment (start 125.36 85.83) (end 124.96 85.83) (width 0.25) (layer F.Cu) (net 25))
 (segment (start 127.06 87.53) (end 125.36 85.83) (width 0.25) (layer F.Cu) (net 25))
 (segment (start 127.16 87.53) (end 127.06 87.53) (width 0.25) (layer F.Cu) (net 25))
 (segment (start 124.96 84.505) (end 125.275 84.19) (width 0.25) (layer F.Cu) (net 25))
 (segment (start 124.96 85.83) (end 124.96 84.505) (width 0.25) (layer F.Cu) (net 25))
 (segment (start 126.875 90.67) (end 126.925 90.72) (width 0.25) (layer F.Cu) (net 25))
 (segment (start 126.875 89.17) (end 126.875 90.67) (width 0.25) (layer F.Cu) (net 25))
 (segment (start 121.1625 87) (end 122.83 87) (width 0.25) (layer F.Cu) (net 30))
 (segment (start 123.36 87.53) (end 124.96 87.53) (width 0.25) (layer F.Cu) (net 30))
 (segment (start 122.83 87) (end 123.36 87.53) (width 0.25) (layer F.Cu) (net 30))
 (segment (start 124.96 88.805) (end 125.325 89.17) (width 0.25) (layer F.Cu) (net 30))
 (segment (start 124.96 87.53) (end 124.96 88.805) (width 0.25) (layer F.Cu) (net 30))
 (segment (start 126.02499 83.38999) (end 126.825 84.19) (width 0.25) (layer F.Cu) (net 29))
 (segment (start 124.822176 83.38999) (end 126.02499 83.38999) (width 0.25) (layer F.Cu) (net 29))
 (segment (start 124.49999 84.32001) (end 124.49999 83.712176) (width 0.25) (layer F.Cu) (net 29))
 (segment (start 122.32 86.5) (end 124.49999 84.32001) (width 0.25) (layer F.Cu) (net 29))
 (segment (start 124.49999 83.712176) (end 124.822176 83.38999) (width 0.25) (layer F.Cu) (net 29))
 (segment (start 121.1625 86.5) (end 122.32 86.5) (width 0.25) (layer F.Cu) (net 29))
 (segment (start 126.825 85.495) (end 127.16 85.83) (width 0.25) (layer F.Cu) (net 29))
 (segment (start 126.825 84.19) (end 126.825 85.495) (width 0.25) (layer F.Cu) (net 29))
 (segment (start 112.33 93.53) (end 112.33 93.92) (width 0.6) (layer F.Cu) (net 28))
 (segment (start 108.170001 89.699999) (end 110.08 91.609998) (width 0.6) (layer F.Cu) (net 28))
 (segment (start 107.045 89.7) (end 108.170001 89.699999) (width 0.6) (layer F.Cu) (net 28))
 (segment (start 110.08 91.609998) (end 110.08 93.52) (width 0.6) (layer F.Cu) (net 28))
 (segment (start 110.48 93.92) (end 112.33 93.92) (width 0.6) (layer F.Cu) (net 28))
 (segment (start 110.08 93.52) (end 110.48 93.92) (width 0.6) (layer F.Cu) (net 28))
 (segment (start 110.22 88.365) (end 110.22 87.62) (width 0.25) (layer F.Cu) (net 22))
 (segment (start 110.22 87.62) (end 110.34 87.5) (width 0.25) (layer F.Cu) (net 22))
 (segment (start 110.34 87.5) (end 112.8375 87.5) (width 0.3) (layer F.Cu) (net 22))
 (segment (start 107.045 87.5) (end 110.34 87.5) (width 0.3) (layer F.Cu) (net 22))
 (segment (start 107.045 87) (end 112.8375 87) (width 0.3) (layer F.Cu) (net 41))
 (segment (start 111.295 90.015) (end 110.22 90.015) (width 0.25) (layer F.Cu) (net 21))
 (segment (start 112.31 89) (end 111.295 90.015) (width 0.25) (layer F.Cu) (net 21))
 (segment (start 112.8375 89) (end 112.31 89) (width 0.25) (layer F.Cu) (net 21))
 (segment (start 119.84 95.7) (end 119.84 97.14) (width 0.25) (layer F.Cu) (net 39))
 (segment (start 119.23 95.09) (end 119.84 95.7) (width 0.25) (layer F.Cu) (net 39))
 (segment (start 118.124298 95.09) (end 119.23 95.09) (width 0.25) (layer F.Cu) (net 39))
 (segment (start 114.25 91.215702) (end 118.124298 95.09) (width 0.25) (layer F.Cu) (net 39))
 (segment (start 114.25 90.4125) (end 114.25 91.215702) (width 0.25) (layer F.Cu) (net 39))
 (segment (start 114.009308 89.34999) (end 113.77499 89.584308) (width 0.25) (layer F.Cu) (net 40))
 (segment (start 114.009308 88.368606) (end 114.009308 89.34999) (width 0.25) (layer F.Cu) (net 40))
 (segment (start 113.77499 89.584308) (end 113.77499 91.377102) (width 0.25) (layer F.Cu) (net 40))
 (segment (start 113.640702 88) (end 114.009308 88.368606) (width 0.25) (layer F.Cu) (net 40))
 (segment (start 112.8375 88) (end 113.640702 88) (width 0.25) (layer F.Cu) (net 40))
 (segment (start 117.84 95.442112) (end 117.84 97.14) (width 0.25) (layer F.Cu) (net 40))
 (segment (start 113.77499 91.377102) (end 117.84 95.442112) (width 0.25) (layer F.Cu) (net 40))
 (segment (start 136.15 89.81) (end 136.23 89.81) (width 0.25) (layer F.Cu) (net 8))
 (segment (start 121.1625 88.5) (end 122.21 88.5) (width 0.25) (layer F.Cu) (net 27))
 (segment (start 124.43 90.72) (end 125.275 90.72) (width 0.25) (layer F.Cu) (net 27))
 (segment (start 122.21 88.5) (end 124.43 90.72) (width 0.25) (layer F.Cu) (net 27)))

